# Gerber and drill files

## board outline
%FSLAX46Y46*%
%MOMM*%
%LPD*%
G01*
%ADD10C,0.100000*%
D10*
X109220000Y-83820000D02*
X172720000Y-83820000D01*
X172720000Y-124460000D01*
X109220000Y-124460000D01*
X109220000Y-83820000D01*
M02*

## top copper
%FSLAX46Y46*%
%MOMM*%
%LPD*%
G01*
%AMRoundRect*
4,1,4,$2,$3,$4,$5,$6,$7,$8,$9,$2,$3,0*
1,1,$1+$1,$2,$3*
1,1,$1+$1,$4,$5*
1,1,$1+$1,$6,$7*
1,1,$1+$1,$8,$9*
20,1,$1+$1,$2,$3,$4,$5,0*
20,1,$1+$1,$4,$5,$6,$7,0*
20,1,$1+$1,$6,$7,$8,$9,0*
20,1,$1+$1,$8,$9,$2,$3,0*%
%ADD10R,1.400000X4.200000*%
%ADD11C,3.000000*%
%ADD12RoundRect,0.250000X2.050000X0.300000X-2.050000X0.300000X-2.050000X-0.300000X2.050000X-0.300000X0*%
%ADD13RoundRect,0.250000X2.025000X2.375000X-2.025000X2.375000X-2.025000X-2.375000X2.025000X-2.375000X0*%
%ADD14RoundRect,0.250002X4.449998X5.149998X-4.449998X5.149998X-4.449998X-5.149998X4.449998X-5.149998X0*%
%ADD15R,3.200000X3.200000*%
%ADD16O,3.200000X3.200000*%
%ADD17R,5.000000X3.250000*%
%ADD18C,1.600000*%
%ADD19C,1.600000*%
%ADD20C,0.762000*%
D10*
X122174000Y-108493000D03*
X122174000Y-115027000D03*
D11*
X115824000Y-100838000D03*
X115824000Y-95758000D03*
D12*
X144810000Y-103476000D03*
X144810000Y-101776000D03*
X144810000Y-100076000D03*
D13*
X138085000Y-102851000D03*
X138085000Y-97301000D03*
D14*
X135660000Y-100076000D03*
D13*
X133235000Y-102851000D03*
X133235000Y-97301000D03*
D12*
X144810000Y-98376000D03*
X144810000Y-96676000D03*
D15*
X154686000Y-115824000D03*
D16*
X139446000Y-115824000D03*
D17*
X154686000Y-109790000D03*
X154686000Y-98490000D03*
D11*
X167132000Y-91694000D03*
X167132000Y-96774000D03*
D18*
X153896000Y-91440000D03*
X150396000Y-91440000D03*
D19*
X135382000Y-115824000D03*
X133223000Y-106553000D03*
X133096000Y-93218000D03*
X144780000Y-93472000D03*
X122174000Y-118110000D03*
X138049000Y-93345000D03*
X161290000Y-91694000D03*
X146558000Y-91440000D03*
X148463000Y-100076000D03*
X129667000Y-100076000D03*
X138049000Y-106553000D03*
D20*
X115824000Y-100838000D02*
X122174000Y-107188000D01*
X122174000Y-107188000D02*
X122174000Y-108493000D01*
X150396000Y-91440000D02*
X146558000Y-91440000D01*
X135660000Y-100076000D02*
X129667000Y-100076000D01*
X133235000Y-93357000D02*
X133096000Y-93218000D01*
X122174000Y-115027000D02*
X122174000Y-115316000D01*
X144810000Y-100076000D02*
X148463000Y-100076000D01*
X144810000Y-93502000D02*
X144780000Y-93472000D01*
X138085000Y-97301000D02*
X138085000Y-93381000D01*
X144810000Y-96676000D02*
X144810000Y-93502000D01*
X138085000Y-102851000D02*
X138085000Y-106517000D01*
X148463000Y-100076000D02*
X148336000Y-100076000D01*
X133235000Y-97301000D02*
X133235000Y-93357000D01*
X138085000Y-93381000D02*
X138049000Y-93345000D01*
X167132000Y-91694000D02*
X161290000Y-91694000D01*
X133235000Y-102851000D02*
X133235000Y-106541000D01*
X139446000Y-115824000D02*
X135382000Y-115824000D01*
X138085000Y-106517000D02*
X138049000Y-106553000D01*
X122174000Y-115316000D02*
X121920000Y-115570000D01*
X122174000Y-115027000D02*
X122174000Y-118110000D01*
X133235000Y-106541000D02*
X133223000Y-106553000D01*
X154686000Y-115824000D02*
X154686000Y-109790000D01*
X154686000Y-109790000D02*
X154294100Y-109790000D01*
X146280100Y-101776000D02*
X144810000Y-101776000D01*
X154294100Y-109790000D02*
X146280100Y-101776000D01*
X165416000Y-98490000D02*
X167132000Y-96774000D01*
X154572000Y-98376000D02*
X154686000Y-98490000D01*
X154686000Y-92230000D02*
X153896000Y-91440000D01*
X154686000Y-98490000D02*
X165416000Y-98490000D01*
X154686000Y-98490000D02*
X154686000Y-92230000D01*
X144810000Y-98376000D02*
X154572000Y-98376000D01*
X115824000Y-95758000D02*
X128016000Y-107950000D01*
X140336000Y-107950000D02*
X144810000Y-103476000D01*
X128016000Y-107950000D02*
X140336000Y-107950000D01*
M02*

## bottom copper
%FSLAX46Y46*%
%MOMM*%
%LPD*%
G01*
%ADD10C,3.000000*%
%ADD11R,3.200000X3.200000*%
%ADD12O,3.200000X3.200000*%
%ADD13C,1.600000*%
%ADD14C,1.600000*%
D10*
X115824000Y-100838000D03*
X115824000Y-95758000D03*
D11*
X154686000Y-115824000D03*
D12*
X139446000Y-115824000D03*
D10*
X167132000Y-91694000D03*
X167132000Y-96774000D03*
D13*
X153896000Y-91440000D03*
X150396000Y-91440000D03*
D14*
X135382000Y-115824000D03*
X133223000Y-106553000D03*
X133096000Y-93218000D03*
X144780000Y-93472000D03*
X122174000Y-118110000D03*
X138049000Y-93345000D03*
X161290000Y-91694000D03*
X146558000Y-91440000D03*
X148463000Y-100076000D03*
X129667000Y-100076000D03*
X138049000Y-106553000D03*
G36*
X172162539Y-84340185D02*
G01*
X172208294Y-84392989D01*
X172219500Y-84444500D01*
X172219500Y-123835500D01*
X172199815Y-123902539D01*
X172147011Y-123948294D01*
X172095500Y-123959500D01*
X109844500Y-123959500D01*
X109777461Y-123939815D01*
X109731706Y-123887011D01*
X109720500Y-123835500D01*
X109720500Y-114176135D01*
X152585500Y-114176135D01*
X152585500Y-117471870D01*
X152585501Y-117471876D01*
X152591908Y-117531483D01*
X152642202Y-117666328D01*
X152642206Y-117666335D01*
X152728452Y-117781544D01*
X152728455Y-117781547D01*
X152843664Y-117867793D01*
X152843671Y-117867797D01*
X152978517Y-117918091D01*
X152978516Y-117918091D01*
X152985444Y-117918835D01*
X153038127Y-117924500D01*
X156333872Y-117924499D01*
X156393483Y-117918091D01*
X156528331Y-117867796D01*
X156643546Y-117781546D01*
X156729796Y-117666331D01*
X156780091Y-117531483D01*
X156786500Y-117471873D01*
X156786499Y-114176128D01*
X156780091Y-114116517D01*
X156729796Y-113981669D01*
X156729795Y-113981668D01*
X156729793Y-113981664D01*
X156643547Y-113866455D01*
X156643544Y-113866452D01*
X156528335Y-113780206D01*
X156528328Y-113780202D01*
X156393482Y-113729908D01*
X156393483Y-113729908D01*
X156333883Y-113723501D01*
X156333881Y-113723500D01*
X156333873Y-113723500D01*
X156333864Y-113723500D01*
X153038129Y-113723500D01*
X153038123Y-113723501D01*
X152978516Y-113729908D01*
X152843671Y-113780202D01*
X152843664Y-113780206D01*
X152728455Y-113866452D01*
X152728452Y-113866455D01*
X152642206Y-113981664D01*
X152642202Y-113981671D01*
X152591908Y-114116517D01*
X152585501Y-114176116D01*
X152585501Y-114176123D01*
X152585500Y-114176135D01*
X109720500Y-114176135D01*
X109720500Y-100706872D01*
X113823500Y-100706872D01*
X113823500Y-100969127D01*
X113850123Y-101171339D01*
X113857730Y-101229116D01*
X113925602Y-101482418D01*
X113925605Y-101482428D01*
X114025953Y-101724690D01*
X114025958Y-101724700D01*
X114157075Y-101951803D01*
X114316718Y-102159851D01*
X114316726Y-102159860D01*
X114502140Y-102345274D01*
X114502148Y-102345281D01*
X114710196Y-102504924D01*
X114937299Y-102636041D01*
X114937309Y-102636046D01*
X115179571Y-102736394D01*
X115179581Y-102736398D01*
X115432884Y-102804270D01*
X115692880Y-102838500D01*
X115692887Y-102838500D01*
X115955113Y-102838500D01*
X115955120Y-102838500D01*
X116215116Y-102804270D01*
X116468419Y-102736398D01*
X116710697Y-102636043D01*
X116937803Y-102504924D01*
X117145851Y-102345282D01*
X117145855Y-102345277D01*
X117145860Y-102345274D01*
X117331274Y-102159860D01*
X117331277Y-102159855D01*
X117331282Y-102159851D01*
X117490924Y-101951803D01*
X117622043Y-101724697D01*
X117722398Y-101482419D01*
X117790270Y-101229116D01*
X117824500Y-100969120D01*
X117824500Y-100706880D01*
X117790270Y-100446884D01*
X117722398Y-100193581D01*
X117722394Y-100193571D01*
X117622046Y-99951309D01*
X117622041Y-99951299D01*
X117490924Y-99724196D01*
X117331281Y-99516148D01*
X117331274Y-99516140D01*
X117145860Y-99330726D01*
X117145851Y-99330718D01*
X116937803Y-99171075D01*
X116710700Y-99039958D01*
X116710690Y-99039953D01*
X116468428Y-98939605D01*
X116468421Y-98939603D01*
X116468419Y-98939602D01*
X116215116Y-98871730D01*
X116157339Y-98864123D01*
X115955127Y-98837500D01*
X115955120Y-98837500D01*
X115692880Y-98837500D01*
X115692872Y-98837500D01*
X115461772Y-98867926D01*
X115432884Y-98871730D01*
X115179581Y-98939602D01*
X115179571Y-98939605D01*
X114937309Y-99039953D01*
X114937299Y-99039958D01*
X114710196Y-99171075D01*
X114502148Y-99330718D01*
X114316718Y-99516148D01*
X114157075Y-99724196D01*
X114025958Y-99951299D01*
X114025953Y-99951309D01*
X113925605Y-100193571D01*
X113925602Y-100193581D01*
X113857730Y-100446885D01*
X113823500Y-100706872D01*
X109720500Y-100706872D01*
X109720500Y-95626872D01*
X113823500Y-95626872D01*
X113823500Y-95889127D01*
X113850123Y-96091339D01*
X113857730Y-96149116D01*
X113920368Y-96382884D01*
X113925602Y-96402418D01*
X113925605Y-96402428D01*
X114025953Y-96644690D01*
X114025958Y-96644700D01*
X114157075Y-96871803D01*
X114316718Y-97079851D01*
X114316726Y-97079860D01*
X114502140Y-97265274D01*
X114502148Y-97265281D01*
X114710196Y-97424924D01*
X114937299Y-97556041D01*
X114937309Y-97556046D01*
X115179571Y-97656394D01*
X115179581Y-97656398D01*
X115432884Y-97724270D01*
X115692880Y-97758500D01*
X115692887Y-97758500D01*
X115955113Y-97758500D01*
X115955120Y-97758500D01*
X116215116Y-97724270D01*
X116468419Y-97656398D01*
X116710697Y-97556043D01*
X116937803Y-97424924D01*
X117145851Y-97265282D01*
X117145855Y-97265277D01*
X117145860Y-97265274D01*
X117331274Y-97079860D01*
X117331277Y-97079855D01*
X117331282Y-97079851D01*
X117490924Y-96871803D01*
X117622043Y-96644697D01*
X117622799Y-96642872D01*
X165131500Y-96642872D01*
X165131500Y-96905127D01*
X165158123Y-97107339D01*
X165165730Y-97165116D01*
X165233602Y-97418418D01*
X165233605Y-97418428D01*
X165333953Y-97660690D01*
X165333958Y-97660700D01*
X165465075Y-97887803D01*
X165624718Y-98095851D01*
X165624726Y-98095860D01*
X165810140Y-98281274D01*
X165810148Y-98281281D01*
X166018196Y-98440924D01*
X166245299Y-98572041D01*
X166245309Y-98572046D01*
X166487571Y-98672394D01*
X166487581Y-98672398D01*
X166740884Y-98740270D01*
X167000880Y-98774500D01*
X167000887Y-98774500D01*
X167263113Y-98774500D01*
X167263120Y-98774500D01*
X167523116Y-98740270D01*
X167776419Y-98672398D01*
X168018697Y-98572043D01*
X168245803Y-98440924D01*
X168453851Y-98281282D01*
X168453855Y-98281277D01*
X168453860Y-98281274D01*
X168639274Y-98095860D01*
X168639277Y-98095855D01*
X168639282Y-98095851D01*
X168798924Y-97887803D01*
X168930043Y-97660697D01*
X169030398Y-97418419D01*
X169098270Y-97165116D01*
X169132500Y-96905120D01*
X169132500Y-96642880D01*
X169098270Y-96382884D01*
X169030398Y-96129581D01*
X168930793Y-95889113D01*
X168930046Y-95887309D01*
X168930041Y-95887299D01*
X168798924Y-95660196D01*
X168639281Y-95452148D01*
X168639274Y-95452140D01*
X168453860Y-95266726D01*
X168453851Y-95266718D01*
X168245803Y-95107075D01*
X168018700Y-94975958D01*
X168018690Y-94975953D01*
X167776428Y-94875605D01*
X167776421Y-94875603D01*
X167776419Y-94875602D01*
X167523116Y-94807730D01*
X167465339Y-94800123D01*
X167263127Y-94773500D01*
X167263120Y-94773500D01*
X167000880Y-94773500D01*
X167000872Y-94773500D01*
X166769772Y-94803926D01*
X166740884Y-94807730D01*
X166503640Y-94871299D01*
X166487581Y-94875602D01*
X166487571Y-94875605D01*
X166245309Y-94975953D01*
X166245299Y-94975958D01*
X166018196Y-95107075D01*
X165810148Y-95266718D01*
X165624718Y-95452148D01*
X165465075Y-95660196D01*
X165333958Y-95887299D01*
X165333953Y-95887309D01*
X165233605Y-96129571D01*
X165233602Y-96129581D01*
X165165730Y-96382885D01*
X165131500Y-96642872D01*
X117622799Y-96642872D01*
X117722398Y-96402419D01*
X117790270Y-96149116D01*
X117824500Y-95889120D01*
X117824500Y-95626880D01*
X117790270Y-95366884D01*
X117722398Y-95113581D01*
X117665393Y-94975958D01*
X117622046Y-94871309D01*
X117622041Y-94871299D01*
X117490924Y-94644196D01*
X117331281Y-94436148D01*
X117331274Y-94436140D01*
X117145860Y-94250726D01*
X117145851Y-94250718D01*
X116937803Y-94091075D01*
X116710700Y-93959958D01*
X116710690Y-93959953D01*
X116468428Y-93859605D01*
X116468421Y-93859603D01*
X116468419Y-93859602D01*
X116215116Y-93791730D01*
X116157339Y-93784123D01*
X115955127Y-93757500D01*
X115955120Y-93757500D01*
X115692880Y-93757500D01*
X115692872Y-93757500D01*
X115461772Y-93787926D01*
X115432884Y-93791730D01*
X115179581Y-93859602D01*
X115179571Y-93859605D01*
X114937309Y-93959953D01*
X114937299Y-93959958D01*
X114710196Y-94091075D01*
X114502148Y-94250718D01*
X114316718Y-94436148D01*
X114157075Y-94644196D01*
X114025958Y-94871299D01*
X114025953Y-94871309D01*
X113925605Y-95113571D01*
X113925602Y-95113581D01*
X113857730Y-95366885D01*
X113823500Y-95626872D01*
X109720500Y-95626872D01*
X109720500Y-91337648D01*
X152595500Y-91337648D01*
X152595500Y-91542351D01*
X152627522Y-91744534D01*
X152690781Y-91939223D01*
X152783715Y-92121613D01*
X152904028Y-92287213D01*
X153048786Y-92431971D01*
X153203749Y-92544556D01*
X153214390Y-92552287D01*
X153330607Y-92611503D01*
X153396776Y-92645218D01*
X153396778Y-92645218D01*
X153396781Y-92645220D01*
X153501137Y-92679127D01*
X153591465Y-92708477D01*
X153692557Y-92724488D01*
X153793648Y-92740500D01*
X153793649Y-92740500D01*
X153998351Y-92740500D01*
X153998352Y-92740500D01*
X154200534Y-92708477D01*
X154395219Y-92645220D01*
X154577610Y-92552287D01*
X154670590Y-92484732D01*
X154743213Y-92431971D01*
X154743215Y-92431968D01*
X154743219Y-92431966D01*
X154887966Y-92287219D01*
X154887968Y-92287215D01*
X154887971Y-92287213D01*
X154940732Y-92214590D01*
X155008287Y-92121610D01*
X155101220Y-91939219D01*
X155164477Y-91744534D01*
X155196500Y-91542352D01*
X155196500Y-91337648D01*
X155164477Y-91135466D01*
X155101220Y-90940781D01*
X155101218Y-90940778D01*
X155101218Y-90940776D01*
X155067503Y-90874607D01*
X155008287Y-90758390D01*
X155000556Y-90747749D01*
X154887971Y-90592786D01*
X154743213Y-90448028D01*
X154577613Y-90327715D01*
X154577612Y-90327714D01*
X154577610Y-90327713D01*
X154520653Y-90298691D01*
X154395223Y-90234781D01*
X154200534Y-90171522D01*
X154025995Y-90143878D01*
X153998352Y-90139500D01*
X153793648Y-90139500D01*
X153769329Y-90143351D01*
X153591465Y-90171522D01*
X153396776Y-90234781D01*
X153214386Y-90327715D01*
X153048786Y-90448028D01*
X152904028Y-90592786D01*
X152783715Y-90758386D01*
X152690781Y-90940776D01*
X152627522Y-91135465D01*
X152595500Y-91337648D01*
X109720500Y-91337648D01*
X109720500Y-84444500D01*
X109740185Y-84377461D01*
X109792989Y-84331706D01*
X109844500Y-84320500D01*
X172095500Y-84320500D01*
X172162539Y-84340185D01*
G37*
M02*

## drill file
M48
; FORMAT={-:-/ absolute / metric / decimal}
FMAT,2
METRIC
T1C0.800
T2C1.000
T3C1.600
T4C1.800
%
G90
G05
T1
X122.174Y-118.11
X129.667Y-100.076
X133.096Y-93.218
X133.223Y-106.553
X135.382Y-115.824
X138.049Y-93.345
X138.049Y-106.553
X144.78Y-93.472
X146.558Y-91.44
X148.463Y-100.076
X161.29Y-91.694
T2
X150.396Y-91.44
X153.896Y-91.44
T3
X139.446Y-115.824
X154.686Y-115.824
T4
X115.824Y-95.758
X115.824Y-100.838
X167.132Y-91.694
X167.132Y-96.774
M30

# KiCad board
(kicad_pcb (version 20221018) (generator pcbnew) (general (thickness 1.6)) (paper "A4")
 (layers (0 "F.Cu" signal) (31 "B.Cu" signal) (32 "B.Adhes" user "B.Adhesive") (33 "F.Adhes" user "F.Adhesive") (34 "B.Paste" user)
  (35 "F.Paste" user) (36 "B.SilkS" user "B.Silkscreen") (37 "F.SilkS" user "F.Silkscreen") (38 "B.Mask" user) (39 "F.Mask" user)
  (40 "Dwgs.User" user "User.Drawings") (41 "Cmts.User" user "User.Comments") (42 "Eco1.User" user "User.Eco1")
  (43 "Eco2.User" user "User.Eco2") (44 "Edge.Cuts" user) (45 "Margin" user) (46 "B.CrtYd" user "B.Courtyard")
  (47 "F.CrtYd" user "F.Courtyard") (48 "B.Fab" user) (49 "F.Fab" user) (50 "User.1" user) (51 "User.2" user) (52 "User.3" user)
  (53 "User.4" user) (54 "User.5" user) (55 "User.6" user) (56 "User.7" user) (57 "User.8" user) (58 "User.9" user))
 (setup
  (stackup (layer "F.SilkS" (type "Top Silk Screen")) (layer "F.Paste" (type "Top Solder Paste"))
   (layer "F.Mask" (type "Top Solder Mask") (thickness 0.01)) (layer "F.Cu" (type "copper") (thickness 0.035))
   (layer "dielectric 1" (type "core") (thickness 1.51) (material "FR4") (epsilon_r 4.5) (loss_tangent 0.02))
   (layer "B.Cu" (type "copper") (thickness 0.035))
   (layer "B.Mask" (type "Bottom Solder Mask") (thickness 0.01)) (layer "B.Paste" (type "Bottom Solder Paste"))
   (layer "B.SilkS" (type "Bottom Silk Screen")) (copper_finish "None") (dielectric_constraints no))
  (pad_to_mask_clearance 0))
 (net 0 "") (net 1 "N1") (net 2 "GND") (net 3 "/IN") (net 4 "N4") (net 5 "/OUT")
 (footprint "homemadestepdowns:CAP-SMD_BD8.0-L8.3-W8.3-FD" (layer "F.Cu") (at 122.174 111.76 -90)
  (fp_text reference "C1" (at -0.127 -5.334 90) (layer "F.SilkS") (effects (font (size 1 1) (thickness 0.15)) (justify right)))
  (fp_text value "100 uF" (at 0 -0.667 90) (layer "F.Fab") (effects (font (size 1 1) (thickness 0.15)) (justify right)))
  (pad "1" smd rect (at -3.267 0 270) (size 4.2 1.4) (layers "F.Cu" "F.Paste" "F.Mask") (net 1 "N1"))
  (pad "2" smd rect (at 3.267 0 270) (size 4.2 1.4) (layers "F.Cu" "F.Paste" "F.Mask") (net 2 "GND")))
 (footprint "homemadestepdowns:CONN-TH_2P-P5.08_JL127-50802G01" (layer "F.Cu") (at 115.824 98.298 90)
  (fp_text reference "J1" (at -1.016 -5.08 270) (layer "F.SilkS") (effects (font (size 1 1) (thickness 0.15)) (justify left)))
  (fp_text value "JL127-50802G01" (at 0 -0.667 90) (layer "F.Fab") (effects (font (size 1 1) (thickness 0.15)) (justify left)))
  (pad "1" thru_hole circle (at -2.54 0 90) (size 3 3) (drill 1.8) (layers "*.Cu" "*.Mask") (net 1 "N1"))
  (pad "2" thru_hole circle (at 2.54 0 90) (size 3 3) (drill 1.8) (layers "*.Cu" "*.Mask") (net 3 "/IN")))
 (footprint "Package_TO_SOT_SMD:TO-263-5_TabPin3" (layer "F.Cu") (at 137.16 100.076 180)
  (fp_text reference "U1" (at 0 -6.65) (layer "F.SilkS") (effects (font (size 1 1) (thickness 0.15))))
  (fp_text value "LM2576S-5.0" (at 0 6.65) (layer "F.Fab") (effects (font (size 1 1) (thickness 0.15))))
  (pad "1" smd roundrect (at -7.65 -3.4 180) (size 4.6 1.1) (layers "F.Cu" "F.Paste" "F.Mask") (roundrect_rratio 0.2272727273) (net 3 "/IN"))
  (pad "2" smd roundrect (at -7.65 -1.7 180) (size 4.6 1.1) (layers "F.Cu" "F.Paste" "F.Mask") (roundrect_rratio 0.2272727273) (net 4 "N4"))
  (pad "3" smd roundrect (at -7.65 0 180) (size 4.6 1.1) (layers "F.Cu" "F.Paste" "F.Mask") (roundrect_rratio 0.2272727273) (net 2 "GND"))
  (pad "3" smd roundrect (at -0.925 -2.775 180) (size 4.55 5.25) (layers "F.Cu" "F.Paste") (roundrect_rratio 0.05494505495) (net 2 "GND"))
  (pad "3" smd roundrect (at -0.925 2.775 180) (size 4.55 5.25) (layers "F.Cu" "F.Paste") (roundrect_rratio 0.05494505495) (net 2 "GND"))
  (pad "3" smd roundrect (at 1.5 0 180) (size 9.4 10.8) (layers "F.Cu" "F.Mask") (roundrect_rratio 0.02659595745) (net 2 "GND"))
  (pad "3" smd roundrect (at 3.925 -2.775 180) (size 4.55 5.25) (layers "F.Cu" "F.Paste") (roundrect_rratio 0.05494505495) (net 2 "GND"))
  (pad "3" smd roundrect (at 3.925 2.775 180) (size 4.55 5.25) (layers "F.Cu" "F.Paste") (roundrect_rratio 0.05494505495) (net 2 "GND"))
  (pad "4" smd roundrect (at -7.65 1.7 180) (size 4.6 1.1) (layers "F.Cu" "F.Paste" "F.Mask") (roundrect_rratio 0.2272727273) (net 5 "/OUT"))
  (pad "5" smd roundrect (at -7.65 3.4 180) (size 4.6 1.1) (layers "F.Cu" "F.Paste" "F.Mask") (roundrect_rratio 0.2272727273) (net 2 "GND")))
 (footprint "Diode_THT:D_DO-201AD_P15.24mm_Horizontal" (layer "F.Cu") (at 154.686 115.824 180)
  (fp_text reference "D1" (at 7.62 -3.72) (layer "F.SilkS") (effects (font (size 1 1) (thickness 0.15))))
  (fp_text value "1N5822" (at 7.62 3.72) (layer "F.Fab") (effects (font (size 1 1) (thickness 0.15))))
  (pad "1" thru_hole rect (at 0 0 180) (size 3.2 3.2) (drill 1.6) (layers "*.Cu" "*.Mask") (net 4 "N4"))
  (pad "2" thru_hole oval (at 15.24 0 180) (size 3.2 3.2) (drill 1.6) (layers "*.Cu" "*.Mask") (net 2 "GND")))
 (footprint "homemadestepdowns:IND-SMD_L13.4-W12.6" (layer "F.Cu") (at 154.686 104.14 90)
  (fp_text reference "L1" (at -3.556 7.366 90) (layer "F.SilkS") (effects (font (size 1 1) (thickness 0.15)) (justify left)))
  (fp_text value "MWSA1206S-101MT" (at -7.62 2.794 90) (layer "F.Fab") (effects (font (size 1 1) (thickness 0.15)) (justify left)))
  (pad "1" smd rect (at -5.65 0 180) (size 5 3.25) (layers "F.Cu" "F.Paste" "F.Mask") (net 4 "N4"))
  (pad "2" smd rect (at 5.65 0 180) (size 5 3.25) (layers "F.Cu" "F.Paste" "F.Mask") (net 5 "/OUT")))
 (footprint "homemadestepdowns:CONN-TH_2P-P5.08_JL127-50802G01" (layer "F.Cu") (at 167.132 94.234 -90)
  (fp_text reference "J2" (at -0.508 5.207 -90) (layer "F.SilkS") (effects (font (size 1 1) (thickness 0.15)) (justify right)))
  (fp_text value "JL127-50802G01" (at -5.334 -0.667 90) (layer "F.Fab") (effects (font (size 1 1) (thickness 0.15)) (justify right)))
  (pad "1" thru_hole circle (at -2.54 0 270) (size 3 3) (drill 1.8) (layers "*.Cu" "*.Mask") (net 2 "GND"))
  (pad "2" thru_hole circle (at 2.54 0 270) (size 3 3) (drill 1.8) (layers "*.Cu" "*.Mask") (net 5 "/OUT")))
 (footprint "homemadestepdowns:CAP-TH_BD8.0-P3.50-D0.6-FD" (layer "F.Cu") (at 152.146 91.44 180)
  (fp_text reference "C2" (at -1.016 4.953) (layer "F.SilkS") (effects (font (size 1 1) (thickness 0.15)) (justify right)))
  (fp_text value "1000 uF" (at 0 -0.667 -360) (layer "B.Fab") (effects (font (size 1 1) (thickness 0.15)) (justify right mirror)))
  (pad "1" thru_hole circle (at -1.75 0 270) (size 1.6 1.6) (drill 1) (layers "*.Cu" "*.Mask") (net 5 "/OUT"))
  (pad "2" thru_hole circle (at 1.75 0 270) (size 1.6 1.6) (drill 1) (layers "*.Cu" "*.Mask") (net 2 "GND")))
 (gr_rect (start 109.22 83.82) (end 172.72 124.46) (stroke (width 0.1) (type default)) (fill none) (layer "Edge.Cuts"))
 (segment (start 115.824 100.838) (end 122.174 107.188) (width 0.762) (layer "F.Cu") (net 1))
 (segment (start 122.174 107.188) (end 122.174 108.493) (width 0.762) (layer "F.Cu") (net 1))
 (segment (start 150.396 91.44) (end 146.558 91.44) (width 0.762) (layer "F.Cu") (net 2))
 (segment (start 135.66 100.076) (end 129.667 100.076) (width 0.762) (layer "F.Cu") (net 2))
 (segment (start 133.235 93.357) (end 133.096 93.218) (width 0.762) (layer "F.Cu") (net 2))
 (segment (start 122.174 115.027) (end 122.174 115.316) (width 0.762) (layer "F.Cu") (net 2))
 (segment (start 144.81 100.076) (end 148.463 100.076) (width 0.762) (layer "F.Cu") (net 2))
 (segment (start 144.81 93.502) (end 144.78 93.472) (width 0.762) (layer "F.Cu") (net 2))
 (segment (start 138.085 97.301) (end 138.085 93.381) (width 0.762) (layer "F.Cu") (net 2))
 (segment (start 144.81 96.676) (end 144.81 93.502) (width 0.762) (layer "F.Cu") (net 2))
 (segment (start 138.085 102.851) (end 138.085 106.517) (width 0.762) (layer "F.Cu") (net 2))
 (segment (start 148.463 100.076) (end 148.336 100.076) (width 0.762) (layer "F.Cu") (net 2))
 (segment (start 133.235 97.301) (end 133.235 93.357) (width 0.762) (layer "F.Cu") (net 2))
 (segment (start 138.085 93.381) (end 138.049 93.345) (width 0.762) (layer "F.Cu") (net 2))
 (segment (start 167.132 91.694) (end 161.29 91.694) (width 0.762) (layer "F.Cu") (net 2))
 (segment (start 133.235 102.851) (end 133.235 106.541) (width 0.762) (layer "F.Cu") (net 2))
 (segment (start 139.446 115.824) (end 135.382 115.824) (width 0.762) (layer "F.Cu") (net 2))
 (segment (start 138.085 106.517) (end 138.049 106.553) (width 0.762) (layer "F.Cu") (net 2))
 (segment (start 122.174 115.316) (end 121.92 115.57) (width 0.762) (layer "F.Cu") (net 2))
 (segment (start 122.174 115.027) (end 122.174 118.11) (width 0.762) (layer "F.Cu") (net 2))
 (segment (start 133.235 106.541) (end 133.223 106.553) (width 0.762) (layer "F.Cu") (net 2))
 (via (at 135.382 115.824) (size 1.6) (drill 0.8) (layers "F.Cu" "B.Cu") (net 2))
 (via (at 133.223 106.553) (size 1.6) (drill 0.8) (layers "F.Cu" "B.Cu") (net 2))
 (via (at 133.096 93.218) (size 1.6) (drill 0.8) (layers "F.Cu" "B.Cu") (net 2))
 (via (at 144.78 93.472) (size 1.6) (drill 0.8) (layers "F.Cu" "B.Cu") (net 2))
 (via (at 122.174 118.11) (size 1.6) (drill 0.8) (layers "F.Cu" "B.Cu") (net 2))
 (via (at 138.049 93.345) (size 1.6) (drill 0.8) (layers "F.Cu" "B.Cu") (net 2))
 (via (at 161.29 91.694) (size 1.6) (drill 0.8) (layers "F.Cu" "B.Cu") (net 2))
 (via (at 146.558 91.44) (size 1.6) (drill 0.8) (layers "F.Cu" "B.Cu") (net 2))
 (via (at 148.463 100.076) (size 1.6) (drill 0.8) (layers "F.Cu" "B.Cu") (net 2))
 (via (at 129.667 100.076) (size 1.6) (drill 0.8) (layers "F.Cu" "B.Cu") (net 2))
 (via (at 138.049 106.553) (size 1.6) (drill 0.8) (layers "F.Cu" "B.Cu") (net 2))
 (segment (start 154.686 115.824) (end 154.686 109.79) (width 0.762) (layer "F.Cu") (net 4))
 (segment (start 154.686 109.79) (end 154.2941 109.79) (width 0.762) (layer "F.Cu") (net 4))
 (segment (start 146.2801 101.776) (end 144.81 101.776) (width 0.762) (layer "F.Cu") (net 4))
 (segment (start 154.2941 109.79) (end 146.2801 101.776) (width 0.762) (layer "F.Cu") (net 4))
 (segment (start 165.416 98.49) (end 167.132 96.774) (width 0.762) (layer "F.Cu") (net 5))
 (segment (start 154.572 98.376) (end 154.686 98.49) (width 0.762) (layer "F.Cu") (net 5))
 (segment (start 154.686 92.23) (end 153.896 91.44) (width 0.762) (layer "F.Cu") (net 5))
 (segment (start 154.686 98.49) (end 165.416 98.49) (width 0.762) (layer "F.Cu") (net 5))
 (segment (start 154.686 98.49) (end 154.686 92.23) (width 0.762) (layer "F.Cu") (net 5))
 (segment (start 144.81 98.376) (end 154.572 98.376) (width 0.762) (layer "F.Cu") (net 5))
 (segment (start 115.824 95.758) (end 128.016 107.95) (width 0.762) (layer "F.Cu") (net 3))
 (segment (start 140.336 107.95) (end 144.81 103.476) (width 0.762) (layer "F.Cu") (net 3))
 (segment (start 128.016 107.95) (end 140.336 107.95) (width 0.762) (layer "F.Cu") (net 3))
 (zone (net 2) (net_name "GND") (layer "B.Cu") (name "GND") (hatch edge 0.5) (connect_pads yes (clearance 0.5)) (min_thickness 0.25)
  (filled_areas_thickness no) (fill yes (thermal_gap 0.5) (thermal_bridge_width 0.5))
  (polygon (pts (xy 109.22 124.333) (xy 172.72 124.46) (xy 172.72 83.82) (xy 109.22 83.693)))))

